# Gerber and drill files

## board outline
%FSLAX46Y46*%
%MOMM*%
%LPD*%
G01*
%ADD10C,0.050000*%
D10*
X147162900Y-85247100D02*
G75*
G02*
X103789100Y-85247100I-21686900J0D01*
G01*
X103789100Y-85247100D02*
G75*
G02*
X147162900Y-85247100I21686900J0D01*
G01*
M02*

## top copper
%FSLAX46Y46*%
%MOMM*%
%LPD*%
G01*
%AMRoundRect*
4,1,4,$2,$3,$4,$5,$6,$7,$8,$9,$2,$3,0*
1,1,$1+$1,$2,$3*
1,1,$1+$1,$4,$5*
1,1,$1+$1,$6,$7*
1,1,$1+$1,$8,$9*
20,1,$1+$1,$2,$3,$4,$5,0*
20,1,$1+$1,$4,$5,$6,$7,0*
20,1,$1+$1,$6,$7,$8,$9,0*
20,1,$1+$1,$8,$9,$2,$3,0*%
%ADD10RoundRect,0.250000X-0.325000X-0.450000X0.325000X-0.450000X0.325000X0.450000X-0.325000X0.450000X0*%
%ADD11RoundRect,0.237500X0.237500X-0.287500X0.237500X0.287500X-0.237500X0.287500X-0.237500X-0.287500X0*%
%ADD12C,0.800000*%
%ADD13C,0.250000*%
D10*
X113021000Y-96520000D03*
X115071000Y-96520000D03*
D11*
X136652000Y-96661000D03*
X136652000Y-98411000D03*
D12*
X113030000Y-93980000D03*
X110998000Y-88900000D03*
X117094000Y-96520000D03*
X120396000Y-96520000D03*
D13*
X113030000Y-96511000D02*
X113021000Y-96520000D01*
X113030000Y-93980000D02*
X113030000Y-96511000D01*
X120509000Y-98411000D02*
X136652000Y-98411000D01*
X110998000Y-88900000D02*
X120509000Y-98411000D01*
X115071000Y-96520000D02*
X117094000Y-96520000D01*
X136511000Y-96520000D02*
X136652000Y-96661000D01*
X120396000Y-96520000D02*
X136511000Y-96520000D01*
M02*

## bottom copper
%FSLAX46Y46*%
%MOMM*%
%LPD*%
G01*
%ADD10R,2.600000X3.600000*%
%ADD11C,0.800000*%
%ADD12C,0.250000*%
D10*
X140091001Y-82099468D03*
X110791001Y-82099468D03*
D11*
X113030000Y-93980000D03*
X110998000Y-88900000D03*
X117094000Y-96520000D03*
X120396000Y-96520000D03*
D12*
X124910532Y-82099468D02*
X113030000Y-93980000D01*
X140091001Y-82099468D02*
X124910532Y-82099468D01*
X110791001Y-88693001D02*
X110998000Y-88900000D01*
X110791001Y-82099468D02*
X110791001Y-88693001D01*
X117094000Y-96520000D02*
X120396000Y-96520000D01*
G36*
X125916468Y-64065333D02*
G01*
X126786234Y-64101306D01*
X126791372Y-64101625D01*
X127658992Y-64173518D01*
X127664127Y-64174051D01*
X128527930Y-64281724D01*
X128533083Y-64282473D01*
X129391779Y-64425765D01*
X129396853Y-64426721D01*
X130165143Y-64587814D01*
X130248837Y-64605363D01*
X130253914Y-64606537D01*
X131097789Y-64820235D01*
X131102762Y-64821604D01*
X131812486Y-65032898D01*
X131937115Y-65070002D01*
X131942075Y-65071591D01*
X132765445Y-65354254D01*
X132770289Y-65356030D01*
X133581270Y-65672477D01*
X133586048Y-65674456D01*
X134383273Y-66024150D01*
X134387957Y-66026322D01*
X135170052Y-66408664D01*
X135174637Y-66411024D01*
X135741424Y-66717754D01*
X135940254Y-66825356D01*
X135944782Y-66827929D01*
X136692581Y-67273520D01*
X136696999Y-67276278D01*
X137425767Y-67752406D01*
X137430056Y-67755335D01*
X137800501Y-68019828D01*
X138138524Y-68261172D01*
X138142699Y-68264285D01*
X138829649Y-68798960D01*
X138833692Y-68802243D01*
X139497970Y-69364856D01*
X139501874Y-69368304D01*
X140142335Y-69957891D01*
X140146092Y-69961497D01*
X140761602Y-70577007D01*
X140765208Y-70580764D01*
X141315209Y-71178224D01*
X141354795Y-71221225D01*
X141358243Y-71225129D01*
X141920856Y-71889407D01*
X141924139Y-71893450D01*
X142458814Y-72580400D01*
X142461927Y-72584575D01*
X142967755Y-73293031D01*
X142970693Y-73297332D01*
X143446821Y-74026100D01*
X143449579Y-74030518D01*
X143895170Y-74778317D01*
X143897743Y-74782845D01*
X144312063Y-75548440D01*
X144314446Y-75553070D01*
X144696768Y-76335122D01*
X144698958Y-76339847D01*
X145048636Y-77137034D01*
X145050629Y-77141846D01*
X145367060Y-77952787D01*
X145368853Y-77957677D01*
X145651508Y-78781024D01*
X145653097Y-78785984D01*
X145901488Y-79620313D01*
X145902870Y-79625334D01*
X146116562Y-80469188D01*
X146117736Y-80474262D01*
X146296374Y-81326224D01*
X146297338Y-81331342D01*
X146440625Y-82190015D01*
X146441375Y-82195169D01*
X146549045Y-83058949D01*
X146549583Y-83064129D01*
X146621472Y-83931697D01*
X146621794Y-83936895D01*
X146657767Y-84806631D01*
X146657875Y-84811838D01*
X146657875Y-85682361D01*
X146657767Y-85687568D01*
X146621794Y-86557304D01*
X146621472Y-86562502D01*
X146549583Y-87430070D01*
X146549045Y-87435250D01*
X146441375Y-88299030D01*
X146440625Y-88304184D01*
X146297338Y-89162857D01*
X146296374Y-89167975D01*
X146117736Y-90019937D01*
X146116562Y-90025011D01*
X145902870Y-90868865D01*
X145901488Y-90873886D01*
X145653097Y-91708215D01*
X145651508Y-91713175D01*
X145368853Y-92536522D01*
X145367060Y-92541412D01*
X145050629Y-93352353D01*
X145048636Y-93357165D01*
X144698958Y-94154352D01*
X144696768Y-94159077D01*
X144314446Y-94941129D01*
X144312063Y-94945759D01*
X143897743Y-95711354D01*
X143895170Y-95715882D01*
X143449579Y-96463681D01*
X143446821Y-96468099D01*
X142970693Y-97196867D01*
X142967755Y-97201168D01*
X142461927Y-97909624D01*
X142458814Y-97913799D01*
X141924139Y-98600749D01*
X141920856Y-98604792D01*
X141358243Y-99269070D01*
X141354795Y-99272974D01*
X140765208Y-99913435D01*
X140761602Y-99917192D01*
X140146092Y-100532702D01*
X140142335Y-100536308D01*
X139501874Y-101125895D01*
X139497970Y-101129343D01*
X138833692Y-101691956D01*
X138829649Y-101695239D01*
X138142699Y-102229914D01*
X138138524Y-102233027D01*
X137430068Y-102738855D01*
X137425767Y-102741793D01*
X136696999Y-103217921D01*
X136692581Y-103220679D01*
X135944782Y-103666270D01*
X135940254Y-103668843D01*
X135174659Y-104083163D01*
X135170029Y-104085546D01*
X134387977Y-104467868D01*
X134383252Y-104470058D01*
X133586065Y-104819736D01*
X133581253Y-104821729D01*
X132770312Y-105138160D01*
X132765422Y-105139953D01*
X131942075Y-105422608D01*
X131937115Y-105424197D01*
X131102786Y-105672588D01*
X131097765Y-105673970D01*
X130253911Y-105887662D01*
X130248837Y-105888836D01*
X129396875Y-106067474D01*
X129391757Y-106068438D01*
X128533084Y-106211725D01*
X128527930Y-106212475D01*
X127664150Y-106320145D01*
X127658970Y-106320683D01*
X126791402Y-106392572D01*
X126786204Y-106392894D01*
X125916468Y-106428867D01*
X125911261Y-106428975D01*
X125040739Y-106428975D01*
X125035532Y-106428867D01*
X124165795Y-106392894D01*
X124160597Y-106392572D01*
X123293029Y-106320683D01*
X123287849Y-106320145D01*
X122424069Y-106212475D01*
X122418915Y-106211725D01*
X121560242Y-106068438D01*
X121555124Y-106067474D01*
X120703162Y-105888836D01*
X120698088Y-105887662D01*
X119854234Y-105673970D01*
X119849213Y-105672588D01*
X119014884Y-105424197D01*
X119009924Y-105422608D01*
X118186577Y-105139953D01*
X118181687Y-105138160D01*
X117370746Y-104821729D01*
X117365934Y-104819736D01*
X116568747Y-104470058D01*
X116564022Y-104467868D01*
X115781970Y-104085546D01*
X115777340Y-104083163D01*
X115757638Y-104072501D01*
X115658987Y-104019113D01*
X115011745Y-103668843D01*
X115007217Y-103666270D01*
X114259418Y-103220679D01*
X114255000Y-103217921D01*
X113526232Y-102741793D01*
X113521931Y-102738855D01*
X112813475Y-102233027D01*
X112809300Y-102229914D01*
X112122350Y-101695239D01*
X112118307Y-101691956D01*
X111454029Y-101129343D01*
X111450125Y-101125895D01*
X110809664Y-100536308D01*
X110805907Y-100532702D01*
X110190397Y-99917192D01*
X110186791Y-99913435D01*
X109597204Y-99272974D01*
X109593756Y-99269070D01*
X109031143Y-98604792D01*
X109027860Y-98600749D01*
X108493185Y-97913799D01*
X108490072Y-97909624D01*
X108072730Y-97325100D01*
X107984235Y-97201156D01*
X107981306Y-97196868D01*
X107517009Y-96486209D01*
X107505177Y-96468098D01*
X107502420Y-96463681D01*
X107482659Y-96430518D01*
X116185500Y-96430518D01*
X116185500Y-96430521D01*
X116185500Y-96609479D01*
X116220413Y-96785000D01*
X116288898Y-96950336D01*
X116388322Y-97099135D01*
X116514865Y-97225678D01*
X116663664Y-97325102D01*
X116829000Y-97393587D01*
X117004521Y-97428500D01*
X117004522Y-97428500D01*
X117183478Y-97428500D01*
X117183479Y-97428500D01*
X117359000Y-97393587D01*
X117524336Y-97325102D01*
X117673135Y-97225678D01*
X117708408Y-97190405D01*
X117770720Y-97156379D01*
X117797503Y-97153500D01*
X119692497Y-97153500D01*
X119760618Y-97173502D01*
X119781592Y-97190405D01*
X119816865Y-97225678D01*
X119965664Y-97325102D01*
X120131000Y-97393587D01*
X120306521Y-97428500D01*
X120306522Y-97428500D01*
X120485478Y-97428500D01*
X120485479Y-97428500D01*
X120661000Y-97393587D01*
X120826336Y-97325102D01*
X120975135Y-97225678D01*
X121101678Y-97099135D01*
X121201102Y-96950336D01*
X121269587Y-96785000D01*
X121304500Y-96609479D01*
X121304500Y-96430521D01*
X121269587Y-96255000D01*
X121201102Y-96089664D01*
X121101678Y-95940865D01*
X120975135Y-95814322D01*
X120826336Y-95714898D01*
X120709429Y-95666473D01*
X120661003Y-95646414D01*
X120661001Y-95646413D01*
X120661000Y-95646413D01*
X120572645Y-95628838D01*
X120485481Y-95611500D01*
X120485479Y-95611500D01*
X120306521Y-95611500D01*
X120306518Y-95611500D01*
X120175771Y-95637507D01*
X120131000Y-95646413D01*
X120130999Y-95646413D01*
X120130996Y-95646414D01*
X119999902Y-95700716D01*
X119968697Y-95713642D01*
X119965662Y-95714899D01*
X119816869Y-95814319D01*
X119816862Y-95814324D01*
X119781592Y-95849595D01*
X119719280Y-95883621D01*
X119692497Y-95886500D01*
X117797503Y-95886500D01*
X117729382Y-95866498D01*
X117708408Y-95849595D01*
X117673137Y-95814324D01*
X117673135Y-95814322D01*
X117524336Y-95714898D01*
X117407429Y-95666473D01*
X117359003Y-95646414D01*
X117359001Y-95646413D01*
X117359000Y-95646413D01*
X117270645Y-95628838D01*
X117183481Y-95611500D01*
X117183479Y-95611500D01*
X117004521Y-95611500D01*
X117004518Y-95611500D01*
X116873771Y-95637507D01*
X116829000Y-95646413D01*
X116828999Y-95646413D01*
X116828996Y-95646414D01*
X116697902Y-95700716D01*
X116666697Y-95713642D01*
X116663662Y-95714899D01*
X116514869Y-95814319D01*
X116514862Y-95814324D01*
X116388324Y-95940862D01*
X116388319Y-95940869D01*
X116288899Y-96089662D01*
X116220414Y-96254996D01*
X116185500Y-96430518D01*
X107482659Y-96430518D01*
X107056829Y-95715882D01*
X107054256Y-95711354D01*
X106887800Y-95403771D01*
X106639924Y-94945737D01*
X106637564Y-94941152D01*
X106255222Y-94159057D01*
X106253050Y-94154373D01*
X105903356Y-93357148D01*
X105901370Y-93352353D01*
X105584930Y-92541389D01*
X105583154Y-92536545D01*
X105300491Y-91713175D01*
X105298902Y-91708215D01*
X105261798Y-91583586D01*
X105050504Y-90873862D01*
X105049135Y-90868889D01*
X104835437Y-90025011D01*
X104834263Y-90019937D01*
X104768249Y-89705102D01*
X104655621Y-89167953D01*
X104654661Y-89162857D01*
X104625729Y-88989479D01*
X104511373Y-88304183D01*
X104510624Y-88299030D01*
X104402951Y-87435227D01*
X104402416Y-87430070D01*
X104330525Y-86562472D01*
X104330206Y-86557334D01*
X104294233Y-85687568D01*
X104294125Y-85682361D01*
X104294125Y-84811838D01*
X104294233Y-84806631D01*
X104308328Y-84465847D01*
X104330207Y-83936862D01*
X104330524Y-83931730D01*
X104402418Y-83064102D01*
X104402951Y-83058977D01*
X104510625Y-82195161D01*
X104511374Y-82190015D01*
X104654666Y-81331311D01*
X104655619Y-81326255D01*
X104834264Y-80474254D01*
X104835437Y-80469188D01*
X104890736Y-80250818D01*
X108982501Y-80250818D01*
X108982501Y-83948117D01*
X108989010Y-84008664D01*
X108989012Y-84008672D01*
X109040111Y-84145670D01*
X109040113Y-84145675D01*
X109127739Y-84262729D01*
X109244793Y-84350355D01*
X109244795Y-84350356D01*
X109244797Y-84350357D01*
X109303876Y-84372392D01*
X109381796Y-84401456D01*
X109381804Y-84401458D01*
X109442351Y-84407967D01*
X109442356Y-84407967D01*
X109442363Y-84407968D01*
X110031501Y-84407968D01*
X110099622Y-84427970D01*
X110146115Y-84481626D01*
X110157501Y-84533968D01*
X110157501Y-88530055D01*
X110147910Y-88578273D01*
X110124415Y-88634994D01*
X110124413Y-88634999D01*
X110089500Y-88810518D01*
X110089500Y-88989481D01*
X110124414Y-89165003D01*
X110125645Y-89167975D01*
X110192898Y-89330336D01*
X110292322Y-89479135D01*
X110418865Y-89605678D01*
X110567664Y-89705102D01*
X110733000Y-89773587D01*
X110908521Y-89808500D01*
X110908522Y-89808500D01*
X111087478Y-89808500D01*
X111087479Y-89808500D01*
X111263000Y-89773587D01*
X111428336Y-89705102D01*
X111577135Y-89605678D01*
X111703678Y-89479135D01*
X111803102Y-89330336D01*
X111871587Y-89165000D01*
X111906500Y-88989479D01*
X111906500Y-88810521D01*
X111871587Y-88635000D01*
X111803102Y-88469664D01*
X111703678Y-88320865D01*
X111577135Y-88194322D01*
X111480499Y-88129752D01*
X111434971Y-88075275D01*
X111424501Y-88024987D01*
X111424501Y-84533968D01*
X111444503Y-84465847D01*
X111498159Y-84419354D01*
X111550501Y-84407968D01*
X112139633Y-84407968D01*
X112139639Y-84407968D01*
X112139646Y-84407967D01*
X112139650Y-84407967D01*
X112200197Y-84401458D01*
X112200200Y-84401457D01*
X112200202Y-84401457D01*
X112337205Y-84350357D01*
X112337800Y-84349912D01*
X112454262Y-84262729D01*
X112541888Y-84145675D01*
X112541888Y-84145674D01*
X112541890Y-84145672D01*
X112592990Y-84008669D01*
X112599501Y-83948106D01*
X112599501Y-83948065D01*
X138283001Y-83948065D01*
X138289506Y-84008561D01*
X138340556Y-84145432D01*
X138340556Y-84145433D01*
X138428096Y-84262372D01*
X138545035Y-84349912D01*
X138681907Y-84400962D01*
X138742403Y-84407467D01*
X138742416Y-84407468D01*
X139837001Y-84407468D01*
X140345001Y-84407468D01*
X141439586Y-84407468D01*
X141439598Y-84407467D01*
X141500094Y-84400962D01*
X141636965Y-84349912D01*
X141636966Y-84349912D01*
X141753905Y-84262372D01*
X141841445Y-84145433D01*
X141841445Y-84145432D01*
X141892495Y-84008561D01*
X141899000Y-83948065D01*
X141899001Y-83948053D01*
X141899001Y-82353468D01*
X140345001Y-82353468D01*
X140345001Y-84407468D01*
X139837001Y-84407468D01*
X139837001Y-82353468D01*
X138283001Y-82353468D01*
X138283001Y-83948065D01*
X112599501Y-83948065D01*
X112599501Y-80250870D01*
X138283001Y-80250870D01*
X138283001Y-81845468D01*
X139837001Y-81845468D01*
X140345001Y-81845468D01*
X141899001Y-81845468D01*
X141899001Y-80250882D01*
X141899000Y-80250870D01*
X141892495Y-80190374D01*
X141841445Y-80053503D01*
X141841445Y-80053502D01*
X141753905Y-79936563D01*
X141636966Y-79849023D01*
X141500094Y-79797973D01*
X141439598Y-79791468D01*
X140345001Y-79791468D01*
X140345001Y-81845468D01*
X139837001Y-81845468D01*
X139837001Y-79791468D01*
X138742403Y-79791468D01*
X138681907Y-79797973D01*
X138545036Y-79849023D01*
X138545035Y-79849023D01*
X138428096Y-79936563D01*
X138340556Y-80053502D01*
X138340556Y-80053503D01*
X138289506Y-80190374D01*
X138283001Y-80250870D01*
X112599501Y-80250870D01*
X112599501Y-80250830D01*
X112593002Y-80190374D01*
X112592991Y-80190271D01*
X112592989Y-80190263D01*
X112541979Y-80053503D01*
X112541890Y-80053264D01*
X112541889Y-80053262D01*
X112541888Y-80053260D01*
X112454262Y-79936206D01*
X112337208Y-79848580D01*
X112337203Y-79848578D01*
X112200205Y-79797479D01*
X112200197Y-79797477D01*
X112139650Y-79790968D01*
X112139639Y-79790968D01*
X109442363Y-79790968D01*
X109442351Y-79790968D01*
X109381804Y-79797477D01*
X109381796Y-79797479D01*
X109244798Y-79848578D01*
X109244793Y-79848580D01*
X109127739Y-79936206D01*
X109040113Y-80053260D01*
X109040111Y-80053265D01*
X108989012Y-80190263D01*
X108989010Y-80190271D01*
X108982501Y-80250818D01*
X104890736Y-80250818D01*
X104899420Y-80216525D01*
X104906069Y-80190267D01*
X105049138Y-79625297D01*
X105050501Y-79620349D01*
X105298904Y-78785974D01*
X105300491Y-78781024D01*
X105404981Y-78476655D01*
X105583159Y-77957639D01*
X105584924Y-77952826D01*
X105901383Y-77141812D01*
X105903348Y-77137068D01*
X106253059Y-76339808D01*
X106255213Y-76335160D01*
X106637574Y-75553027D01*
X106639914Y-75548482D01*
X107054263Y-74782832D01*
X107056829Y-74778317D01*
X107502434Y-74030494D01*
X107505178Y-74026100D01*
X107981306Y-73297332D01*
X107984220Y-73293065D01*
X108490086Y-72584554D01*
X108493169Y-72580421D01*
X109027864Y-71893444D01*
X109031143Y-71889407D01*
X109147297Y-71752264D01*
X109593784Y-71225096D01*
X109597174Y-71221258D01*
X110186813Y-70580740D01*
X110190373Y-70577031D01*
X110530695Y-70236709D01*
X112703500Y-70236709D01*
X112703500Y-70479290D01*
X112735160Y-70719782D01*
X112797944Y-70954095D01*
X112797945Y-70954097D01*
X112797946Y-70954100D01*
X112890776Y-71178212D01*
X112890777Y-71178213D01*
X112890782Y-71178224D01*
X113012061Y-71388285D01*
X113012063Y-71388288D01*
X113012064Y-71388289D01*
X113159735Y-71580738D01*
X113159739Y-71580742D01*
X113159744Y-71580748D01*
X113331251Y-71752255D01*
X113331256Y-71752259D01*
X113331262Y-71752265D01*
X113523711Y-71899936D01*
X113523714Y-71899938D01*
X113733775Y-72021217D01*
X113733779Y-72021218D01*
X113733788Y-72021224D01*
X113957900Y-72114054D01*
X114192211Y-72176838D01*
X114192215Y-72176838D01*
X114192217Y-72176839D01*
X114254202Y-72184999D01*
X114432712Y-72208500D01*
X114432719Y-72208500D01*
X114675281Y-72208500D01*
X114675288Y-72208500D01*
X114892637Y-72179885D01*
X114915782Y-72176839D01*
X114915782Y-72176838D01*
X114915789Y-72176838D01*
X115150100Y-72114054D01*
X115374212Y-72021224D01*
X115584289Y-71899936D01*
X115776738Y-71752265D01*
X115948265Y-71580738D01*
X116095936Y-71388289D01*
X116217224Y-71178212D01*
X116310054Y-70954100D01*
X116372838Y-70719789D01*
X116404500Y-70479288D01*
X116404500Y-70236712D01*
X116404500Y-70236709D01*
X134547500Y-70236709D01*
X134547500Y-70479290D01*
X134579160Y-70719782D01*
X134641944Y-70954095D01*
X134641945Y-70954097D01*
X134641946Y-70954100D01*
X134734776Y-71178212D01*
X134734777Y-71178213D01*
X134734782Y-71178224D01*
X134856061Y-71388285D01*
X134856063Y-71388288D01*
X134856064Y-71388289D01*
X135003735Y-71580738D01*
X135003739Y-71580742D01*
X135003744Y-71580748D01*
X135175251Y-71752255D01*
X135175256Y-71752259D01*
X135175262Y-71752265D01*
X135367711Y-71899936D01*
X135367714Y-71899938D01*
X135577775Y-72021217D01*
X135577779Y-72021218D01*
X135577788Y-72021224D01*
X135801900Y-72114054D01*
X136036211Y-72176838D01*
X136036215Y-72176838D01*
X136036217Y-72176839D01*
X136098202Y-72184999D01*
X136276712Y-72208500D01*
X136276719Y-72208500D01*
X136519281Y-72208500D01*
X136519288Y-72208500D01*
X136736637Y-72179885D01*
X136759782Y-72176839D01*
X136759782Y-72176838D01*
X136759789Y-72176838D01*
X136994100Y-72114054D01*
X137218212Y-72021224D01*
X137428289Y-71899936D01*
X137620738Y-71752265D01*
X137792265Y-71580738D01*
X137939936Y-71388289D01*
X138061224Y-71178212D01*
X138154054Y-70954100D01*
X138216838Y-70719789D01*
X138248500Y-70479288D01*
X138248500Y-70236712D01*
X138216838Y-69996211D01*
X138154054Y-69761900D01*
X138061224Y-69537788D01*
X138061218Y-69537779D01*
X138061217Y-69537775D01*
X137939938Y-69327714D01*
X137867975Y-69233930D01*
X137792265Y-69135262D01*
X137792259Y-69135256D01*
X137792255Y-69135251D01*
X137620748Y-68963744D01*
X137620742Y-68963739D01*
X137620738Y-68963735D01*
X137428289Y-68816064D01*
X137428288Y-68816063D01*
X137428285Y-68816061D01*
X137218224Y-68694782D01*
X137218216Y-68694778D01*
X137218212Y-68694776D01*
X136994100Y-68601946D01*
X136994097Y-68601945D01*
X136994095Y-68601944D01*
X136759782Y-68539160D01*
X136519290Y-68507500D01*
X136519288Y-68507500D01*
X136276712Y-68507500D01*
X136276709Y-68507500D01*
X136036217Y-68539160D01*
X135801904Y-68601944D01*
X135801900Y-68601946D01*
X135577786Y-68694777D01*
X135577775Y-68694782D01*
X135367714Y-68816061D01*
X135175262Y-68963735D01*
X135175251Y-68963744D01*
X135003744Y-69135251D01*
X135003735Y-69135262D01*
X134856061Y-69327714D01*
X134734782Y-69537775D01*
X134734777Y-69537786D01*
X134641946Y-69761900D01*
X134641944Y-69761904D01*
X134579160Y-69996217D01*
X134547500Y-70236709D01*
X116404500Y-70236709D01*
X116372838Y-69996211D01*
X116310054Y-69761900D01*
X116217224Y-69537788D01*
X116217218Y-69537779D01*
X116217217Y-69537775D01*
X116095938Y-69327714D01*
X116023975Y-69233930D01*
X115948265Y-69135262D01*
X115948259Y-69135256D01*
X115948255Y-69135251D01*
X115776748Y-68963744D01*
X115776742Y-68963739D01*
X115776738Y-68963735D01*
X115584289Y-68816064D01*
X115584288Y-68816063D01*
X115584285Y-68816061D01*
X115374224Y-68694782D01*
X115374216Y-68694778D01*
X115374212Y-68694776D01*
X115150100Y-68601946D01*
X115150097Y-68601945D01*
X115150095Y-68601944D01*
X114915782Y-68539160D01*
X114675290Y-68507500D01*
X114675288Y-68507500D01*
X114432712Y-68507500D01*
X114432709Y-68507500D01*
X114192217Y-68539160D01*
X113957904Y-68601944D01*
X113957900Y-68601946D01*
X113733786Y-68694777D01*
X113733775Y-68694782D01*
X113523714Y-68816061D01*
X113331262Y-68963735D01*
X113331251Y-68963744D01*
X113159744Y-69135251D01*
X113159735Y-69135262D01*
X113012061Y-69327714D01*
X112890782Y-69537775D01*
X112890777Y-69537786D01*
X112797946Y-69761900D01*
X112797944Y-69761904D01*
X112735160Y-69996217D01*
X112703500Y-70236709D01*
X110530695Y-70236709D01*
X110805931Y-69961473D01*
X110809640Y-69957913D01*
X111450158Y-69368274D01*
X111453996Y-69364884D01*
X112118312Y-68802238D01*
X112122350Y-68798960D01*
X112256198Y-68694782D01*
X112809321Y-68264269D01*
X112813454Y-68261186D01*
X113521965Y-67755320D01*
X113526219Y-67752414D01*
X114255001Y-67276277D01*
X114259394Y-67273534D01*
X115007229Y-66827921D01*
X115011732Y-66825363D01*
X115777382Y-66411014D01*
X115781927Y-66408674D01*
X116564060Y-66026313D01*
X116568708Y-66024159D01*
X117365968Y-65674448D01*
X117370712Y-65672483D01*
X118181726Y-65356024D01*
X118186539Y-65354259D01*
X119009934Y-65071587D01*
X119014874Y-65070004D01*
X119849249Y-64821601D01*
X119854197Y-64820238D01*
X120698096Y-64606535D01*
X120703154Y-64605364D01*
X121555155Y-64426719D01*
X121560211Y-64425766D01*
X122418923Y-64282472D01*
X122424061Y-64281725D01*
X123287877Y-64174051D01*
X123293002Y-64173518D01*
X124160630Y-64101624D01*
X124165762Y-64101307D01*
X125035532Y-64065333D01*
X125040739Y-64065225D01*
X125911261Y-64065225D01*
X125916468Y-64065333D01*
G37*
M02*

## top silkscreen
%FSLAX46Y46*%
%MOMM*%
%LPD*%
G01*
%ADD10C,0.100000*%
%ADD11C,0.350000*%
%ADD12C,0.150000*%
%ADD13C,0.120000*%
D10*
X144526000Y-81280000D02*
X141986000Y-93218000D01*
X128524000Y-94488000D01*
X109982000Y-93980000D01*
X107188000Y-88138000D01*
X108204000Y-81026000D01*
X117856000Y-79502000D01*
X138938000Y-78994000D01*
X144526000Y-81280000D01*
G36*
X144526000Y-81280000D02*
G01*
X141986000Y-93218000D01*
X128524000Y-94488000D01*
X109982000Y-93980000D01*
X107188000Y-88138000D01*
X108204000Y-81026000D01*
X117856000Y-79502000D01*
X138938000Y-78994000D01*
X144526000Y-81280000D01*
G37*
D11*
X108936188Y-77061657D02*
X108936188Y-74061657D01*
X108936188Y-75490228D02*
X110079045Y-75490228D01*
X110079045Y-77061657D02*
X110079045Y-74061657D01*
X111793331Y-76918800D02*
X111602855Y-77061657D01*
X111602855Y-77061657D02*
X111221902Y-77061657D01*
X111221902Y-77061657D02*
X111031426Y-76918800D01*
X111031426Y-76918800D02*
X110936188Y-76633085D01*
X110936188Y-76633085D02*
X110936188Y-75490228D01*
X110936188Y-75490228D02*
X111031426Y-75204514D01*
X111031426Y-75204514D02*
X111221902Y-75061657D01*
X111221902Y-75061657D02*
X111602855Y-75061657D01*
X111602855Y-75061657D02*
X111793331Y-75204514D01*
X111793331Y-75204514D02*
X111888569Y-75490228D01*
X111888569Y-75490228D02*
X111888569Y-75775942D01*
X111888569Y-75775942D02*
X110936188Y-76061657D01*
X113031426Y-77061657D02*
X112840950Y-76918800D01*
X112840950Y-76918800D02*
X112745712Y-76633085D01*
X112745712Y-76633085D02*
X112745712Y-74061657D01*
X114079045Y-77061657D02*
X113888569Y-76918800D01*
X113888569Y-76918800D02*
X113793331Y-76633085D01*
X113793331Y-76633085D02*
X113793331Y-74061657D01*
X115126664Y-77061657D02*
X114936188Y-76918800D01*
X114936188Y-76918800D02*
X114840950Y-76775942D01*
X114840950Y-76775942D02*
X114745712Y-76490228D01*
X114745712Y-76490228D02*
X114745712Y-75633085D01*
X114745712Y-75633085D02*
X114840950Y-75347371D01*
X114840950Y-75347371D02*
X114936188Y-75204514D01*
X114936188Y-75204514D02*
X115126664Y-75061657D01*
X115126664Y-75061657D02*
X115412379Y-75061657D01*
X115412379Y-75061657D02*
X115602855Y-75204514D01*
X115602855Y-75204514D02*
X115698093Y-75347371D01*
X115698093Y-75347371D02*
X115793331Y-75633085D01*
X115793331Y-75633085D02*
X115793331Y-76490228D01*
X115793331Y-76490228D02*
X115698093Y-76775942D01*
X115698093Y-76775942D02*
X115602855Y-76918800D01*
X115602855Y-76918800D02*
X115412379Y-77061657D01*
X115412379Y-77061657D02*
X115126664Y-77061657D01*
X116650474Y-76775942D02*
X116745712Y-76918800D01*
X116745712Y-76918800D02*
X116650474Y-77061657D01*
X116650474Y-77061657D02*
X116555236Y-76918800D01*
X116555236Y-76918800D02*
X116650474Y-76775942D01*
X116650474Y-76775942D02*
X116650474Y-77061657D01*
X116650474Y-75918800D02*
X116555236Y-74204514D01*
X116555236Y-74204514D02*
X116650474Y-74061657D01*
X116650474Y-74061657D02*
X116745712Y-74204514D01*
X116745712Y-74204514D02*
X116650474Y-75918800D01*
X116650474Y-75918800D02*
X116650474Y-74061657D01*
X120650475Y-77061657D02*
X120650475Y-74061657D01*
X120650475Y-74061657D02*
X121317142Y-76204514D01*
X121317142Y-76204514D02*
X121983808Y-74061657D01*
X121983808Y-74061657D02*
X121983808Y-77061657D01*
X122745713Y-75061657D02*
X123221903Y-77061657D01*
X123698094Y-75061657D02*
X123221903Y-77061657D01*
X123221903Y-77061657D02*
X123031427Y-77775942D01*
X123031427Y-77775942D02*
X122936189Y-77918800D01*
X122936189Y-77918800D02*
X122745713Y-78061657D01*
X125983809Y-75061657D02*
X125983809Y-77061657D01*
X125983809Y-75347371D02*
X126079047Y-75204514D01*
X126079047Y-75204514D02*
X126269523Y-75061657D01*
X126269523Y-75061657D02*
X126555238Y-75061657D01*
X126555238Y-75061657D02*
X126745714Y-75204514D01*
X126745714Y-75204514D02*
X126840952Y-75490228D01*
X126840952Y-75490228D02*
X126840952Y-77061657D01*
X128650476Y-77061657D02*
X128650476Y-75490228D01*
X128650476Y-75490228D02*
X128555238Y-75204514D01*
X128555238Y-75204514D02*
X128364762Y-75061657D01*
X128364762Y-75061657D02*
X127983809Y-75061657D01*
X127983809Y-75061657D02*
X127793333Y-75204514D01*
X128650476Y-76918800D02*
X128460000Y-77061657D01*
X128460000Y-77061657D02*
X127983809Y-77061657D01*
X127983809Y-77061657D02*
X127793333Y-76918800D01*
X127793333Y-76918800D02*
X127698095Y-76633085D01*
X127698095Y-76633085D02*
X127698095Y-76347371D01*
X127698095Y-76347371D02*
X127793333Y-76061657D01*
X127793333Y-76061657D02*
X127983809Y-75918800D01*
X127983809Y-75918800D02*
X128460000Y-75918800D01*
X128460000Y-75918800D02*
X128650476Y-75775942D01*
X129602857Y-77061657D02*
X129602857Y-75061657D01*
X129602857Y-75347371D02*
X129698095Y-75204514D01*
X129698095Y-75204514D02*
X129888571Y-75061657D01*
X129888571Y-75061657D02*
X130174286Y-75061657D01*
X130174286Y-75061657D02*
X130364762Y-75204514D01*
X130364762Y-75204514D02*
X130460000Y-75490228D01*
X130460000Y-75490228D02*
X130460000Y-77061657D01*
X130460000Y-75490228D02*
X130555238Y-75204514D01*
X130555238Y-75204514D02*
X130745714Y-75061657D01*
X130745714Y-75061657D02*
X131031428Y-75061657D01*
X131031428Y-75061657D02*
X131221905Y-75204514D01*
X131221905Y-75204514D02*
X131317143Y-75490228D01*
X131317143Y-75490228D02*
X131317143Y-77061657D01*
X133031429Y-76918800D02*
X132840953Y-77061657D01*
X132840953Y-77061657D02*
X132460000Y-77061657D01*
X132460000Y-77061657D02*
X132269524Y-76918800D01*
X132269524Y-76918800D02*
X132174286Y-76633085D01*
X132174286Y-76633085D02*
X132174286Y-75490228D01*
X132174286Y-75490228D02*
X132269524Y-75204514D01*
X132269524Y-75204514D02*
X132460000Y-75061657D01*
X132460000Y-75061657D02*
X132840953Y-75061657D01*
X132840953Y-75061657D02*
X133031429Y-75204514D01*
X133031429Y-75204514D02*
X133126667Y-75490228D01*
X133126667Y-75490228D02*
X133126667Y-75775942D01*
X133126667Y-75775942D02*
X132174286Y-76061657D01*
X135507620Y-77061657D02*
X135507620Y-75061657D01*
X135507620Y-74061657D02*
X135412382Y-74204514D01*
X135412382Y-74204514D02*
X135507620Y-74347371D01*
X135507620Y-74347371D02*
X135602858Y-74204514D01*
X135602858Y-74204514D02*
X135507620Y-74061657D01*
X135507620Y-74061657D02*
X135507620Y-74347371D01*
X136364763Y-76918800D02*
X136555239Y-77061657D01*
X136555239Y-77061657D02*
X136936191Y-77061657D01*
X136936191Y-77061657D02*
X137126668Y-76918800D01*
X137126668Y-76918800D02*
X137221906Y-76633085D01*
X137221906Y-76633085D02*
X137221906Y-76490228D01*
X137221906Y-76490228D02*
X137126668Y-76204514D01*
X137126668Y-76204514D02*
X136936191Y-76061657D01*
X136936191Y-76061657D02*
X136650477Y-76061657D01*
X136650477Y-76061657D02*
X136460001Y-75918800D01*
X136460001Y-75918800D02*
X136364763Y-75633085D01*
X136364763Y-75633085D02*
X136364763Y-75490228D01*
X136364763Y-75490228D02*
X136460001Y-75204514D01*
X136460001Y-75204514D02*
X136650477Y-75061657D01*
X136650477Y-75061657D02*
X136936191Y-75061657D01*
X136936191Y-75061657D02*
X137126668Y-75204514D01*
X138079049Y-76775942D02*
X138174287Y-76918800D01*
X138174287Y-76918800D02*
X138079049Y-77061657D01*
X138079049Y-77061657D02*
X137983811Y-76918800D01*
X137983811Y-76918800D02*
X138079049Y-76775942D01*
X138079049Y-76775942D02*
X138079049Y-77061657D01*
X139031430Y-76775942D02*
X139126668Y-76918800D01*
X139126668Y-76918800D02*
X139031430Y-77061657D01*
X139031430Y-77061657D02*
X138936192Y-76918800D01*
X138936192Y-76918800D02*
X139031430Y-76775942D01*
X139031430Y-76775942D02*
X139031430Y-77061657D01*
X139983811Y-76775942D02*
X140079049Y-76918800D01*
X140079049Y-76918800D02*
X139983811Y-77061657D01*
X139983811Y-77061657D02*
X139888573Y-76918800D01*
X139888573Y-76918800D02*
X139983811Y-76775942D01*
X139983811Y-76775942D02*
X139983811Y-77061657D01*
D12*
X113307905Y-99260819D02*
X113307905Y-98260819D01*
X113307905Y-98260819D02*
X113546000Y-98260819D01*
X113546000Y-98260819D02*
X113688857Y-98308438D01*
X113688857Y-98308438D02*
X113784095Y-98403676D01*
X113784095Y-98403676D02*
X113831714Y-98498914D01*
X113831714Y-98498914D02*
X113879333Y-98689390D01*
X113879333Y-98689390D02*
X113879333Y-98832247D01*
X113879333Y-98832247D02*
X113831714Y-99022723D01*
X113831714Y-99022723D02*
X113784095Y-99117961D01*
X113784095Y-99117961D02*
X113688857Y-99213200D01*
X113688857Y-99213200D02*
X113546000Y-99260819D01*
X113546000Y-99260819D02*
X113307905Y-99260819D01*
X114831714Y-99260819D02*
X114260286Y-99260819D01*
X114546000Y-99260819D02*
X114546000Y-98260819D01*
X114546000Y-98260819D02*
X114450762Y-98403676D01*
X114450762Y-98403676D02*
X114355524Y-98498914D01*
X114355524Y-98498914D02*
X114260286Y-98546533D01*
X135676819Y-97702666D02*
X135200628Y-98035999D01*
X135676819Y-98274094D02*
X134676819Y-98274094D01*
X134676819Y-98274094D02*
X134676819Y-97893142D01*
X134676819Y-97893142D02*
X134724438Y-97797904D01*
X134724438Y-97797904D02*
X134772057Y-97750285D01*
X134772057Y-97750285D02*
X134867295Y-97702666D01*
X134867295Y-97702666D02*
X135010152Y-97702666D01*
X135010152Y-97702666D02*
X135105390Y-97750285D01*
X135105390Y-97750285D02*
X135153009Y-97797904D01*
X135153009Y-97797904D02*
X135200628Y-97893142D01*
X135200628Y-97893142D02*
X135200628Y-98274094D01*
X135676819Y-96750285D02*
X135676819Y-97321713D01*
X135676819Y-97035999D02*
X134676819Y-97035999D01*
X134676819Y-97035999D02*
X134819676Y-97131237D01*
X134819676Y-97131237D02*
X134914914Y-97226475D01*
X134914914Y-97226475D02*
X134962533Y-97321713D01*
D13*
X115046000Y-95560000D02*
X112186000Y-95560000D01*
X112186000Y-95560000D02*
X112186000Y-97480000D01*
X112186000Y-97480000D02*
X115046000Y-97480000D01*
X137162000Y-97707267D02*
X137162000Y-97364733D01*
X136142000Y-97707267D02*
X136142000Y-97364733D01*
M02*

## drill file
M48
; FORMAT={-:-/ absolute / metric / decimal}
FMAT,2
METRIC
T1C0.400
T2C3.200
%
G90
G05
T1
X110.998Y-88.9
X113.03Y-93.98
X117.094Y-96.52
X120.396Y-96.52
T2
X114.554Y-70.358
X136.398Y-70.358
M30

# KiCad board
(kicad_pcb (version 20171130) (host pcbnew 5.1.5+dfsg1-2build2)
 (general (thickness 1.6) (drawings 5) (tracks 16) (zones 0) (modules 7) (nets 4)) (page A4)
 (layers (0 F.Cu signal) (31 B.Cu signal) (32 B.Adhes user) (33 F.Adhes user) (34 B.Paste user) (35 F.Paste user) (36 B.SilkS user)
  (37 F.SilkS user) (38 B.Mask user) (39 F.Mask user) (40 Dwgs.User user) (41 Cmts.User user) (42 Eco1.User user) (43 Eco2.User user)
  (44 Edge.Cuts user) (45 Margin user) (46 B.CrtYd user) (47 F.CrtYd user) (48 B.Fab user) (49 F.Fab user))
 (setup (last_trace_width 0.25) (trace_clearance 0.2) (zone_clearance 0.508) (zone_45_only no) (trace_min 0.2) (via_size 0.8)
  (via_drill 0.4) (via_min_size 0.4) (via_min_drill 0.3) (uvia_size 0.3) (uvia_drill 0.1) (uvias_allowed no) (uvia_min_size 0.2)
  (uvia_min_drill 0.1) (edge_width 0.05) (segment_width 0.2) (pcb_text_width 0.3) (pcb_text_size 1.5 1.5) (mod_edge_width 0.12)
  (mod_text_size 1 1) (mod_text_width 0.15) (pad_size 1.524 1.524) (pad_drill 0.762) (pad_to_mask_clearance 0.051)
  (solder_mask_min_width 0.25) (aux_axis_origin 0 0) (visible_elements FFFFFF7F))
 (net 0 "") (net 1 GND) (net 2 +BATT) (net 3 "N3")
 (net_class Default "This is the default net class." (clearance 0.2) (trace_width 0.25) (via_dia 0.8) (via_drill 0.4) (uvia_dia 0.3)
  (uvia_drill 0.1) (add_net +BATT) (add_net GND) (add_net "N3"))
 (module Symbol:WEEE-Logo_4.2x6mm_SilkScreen (layer B.Cu) (at 122.428 69.088 180)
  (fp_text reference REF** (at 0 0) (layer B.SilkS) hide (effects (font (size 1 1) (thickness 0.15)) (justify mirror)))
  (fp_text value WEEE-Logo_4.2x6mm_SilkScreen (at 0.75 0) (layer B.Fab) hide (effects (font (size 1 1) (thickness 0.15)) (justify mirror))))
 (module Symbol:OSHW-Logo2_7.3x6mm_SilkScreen (layer B.Cu) (at 129.286 69.342 180)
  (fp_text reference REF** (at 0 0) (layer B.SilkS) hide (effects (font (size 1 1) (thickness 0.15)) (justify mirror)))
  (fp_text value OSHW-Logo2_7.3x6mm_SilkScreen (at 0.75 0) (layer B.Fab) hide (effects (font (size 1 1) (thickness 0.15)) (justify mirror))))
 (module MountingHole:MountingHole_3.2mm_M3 (layer F.Cu) (at 136.398 70.358)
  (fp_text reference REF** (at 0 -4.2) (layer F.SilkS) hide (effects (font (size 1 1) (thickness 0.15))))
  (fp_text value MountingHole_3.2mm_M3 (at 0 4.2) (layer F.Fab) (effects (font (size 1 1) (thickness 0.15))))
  (pad 1 np_thru_hole circle (at 0 0) (size 3.2 3.2) (drill 3.2) (layers *.Cu *.Mask)))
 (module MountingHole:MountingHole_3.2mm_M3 (layer F.Cu) (at 114.554 70.358)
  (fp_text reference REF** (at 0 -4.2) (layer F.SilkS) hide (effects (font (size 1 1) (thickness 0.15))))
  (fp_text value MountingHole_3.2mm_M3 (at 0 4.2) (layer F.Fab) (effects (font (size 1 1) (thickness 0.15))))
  (pad 1 np_thru_hole circle (at 0 0) (size 3.2 3.2) (drill 3.2) (layers *.Cu *.Mask)))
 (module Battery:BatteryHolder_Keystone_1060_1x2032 (layer B.Cu) (at 125.441001 82.099468)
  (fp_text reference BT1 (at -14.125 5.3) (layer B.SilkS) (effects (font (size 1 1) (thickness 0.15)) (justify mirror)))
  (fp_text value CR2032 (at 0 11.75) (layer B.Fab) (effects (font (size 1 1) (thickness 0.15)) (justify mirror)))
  (pad 2 smd rect (at 14.65 0 180) (size 2.6 3.6) (layers B.Cu B.Paste B.Mask) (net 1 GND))
  (pad 1 smd rect (at -14.65 0 180) (size 2.6 3.6) (layers B.Cu B.Paste B.Mask) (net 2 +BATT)))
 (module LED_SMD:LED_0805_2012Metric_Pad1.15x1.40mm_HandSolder (layer F.Cu) (at 114.046 96.52)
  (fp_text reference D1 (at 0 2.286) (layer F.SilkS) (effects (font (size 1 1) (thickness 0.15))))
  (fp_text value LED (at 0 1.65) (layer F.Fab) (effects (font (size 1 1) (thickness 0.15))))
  (fp_line (start 1 -0.96) (end -1.86 -0.96) (layer F.SilkS) (width 0.12))
  (fp_line (start -1.86 -0.96) (end -1.86 0.96) (layer F.SilkS) (width 0.12))
  (fp_line (start -1.86 0.96) (end 1 0.96) (layer F.SilkS) (width 0.12))
  (pad 1 smd roundrect (at -1.025 0) (size 1.15 1.4) (layers F.Cu F.Paste F.Mask) (roundrect_rratio 0.217391) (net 1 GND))
  (pad 2 smd roundrect (at 1.025 0) (size 1.15 1.4) (layers F.Cu F.Paste F.Mask) (roundrect_rratio 0.217391) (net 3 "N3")))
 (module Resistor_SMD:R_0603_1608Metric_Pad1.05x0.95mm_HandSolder (layer F.Cu) (at 136.652 97.536 90)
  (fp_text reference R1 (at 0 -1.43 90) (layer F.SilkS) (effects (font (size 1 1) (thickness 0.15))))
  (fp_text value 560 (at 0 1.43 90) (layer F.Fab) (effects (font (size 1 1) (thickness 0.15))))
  (fp_line (start -0.171267 0.51) (end 0.171267 0.51) (layer F.SilkS) (width 0.12))
  (fp_line (start -0.171267 -0.51) (end 0.171267 -0.51) (layer F.SilkS) (width 0.12))
  (pad 2 smd roundrect (at 0.875 0 90) (size 1.05 0.95) (layers F.Cu F.Paste F.Mask) (roundrect_rratio 0.25) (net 3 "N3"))
  (pad 1 smd roundrect (at -0.875 0 90) (size 1.05 0.95) (layers F.Cu F.Paste F.Mask) (roundrect_rratio 0.25) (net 2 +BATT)))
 (gr_poly
  (pts (xy 144.526 81.28) (xy 141.986 93.218) (xy 128.524 94.488) (xy 109.982 93.98) (xy 107.188 88.138) (xy 108.204 81.026)
   (xy 117.856 79.502) (xy 138.938 78.994))
  (layer F.SilkS) (width 0.1))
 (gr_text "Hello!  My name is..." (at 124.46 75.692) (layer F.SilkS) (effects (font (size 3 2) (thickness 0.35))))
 (gr_circle (center 125.476 85.2471) (end 146.05 92.1051) (layer Edge.Cuts) (width 0.05))
 (via (at 113.03 93.98) (size 0.8) (drill 0.4) (layers F.Cu B.Cu) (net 1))
 (segment (start 124.910532 82.099468) (end 113.03 93.98) (width 0.25) (layer B.Cu) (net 1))
 (segment (start 140.091001 82.099468) (end 124.910532 82.099468) (width 0.25) (layer B.Cu) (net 1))
 (segment (start 113.03 96.511) (end 113.021 96.52) (width 0.25) (layer F.Cu) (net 1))
 (segment (start 113.03 93.98) (end 113.03 96.511) (width 0.25) (layer F.Cu) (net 1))
 (via (at 110.998 88.9) (size 0.8) (drill 0.4) (layers F.Cu B.Cu) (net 2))
 (segment (start 110.791001 88.693001) (end 110.998 88.9) (width 0.25) (layer B.Cu) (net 2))
 (segment (start 110.791001 82.099468) (end 110.791001 88.693001) (width 0.25) (layer B.Cu) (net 2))
 (segment (start 120.509 98.411) (end 136.652 98.411) (width 0.25) (layer F.Cu) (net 2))
 (segment (start 110.998 88.9) (end 120.509 98.411) (width 0.25) (layer F.Cu) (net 2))
 (via (at 117.094 96.52) (size 0.8) (drill 0.4) (layers F.Cu B.Cu) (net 3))
 (segment (start 115.071 96.52) (end 117.094 96.52) (width 0.25) (layer F.Cu) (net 3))
 (via (at 120.396 96.52) (size 0.8) (drill 0.4) (layers F.Cu B.Cu) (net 3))
 (segment (start 117.094 96.52) (end 120.396 96.52) (width 0.25) (layer B.Cu) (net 3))
 (segment (start 136.511 96.52) (end 136.652 96.661) (width 0.25) (layer F.Cu) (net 3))
 (segment (start 120.396 96.52) (end 136.511 96.52) (width 0.25) (layer F.Cu) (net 3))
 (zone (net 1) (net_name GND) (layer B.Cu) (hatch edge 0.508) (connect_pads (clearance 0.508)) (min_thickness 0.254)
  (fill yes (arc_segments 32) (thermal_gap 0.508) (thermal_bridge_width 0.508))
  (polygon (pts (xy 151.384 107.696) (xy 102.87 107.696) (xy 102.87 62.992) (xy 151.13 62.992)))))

